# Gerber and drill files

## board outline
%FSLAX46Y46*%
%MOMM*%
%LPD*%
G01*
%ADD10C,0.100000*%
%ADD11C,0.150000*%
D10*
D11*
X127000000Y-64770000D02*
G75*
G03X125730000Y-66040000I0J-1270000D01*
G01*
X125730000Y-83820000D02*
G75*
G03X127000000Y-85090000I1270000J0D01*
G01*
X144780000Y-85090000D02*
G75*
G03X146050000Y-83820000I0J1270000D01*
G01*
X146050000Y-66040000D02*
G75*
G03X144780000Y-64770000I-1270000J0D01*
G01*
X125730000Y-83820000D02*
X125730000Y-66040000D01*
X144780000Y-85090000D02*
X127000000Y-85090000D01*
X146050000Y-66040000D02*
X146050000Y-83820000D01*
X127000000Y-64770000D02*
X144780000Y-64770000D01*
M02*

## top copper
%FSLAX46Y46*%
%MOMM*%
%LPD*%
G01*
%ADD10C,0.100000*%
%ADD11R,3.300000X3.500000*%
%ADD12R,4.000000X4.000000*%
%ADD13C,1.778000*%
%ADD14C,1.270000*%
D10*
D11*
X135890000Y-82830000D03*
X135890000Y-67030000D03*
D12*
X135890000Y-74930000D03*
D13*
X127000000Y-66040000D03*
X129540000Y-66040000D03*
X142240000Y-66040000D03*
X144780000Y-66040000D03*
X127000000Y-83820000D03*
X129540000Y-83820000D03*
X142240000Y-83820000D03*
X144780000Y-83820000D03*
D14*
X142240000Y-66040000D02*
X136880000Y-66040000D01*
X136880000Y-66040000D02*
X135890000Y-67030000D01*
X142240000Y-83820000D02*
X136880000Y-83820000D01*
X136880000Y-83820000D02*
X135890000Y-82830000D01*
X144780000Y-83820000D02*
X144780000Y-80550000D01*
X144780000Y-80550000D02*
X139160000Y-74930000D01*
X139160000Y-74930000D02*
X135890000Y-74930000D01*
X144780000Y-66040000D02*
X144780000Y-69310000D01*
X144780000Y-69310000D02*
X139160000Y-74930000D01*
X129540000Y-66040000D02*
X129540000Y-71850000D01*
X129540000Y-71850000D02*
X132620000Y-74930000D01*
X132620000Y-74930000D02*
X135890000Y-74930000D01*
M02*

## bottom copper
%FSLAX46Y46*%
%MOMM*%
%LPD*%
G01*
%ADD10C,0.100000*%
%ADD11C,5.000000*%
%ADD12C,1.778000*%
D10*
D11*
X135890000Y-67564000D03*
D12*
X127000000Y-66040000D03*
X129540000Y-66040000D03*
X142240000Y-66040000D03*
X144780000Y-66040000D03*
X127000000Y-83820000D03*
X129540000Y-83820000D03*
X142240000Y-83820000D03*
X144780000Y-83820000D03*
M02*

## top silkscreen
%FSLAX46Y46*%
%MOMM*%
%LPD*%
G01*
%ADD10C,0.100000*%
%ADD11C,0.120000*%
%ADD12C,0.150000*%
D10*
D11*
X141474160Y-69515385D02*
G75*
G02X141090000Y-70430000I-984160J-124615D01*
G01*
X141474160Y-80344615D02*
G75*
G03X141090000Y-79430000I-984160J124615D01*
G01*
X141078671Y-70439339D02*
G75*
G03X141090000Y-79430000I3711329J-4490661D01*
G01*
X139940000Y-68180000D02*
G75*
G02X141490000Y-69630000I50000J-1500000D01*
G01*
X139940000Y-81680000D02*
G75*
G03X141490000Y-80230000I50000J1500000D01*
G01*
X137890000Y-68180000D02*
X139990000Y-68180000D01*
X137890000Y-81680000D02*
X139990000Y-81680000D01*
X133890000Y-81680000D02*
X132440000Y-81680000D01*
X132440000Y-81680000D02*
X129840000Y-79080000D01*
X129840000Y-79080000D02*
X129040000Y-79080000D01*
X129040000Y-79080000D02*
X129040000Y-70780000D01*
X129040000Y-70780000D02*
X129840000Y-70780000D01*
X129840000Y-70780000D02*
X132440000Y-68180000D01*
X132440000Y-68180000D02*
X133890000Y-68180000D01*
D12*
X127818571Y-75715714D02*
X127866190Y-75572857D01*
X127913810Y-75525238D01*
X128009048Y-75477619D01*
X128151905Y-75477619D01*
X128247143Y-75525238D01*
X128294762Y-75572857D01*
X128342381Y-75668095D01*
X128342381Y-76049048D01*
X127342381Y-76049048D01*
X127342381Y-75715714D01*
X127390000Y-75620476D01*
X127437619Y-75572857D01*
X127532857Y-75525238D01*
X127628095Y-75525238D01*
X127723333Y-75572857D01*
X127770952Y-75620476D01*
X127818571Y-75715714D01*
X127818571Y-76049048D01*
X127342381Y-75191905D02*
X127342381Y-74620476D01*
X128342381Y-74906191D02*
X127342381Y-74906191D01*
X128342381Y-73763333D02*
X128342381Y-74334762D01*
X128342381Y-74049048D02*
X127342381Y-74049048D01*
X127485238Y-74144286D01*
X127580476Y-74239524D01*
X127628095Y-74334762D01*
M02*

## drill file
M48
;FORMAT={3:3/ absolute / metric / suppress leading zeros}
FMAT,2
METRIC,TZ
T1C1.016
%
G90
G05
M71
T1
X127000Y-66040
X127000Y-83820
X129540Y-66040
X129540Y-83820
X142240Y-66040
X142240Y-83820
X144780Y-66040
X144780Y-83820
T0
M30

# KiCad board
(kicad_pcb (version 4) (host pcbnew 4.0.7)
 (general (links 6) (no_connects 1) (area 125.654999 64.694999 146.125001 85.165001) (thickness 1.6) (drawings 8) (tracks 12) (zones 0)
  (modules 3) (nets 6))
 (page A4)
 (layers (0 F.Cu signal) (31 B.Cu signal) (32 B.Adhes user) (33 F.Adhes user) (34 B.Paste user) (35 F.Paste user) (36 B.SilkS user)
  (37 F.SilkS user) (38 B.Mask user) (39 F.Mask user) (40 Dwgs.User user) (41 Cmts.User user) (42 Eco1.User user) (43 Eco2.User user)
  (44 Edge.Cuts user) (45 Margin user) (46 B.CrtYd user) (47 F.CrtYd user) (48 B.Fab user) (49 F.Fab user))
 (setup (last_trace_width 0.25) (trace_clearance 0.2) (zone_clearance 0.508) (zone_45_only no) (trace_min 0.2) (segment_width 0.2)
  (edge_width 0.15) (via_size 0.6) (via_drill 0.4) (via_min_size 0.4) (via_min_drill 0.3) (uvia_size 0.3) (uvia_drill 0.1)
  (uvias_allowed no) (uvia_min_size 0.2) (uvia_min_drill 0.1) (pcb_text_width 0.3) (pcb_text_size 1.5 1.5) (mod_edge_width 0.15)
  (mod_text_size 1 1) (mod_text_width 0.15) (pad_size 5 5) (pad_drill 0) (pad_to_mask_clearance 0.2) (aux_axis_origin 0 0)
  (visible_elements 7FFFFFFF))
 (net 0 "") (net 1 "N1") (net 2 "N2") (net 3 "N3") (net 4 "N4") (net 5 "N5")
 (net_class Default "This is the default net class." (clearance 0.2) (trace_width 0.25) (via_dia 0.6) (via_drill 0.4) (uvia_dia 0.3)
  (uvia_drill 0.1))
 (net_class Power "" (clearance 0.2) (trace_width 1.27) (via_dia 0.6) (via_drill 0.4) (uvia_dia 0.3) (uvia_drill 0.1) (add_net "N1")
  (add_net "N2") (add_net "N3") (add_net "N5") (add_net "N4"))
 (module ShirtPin (layer B.Cu) (at 135.89 67.564)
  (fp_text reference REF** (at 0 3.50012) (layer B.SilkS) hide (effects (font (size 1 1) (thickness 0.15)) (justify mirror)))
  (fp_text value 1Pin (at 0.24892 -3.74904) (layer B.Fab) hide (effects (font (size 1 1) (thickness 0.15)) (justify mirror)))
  (pad 1 smd circle (at 0 0) (size 5 5) (layers B.Cu B.Mask)))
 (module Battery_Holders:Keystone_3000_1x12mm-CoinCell (layer F.Cu) (at 135.89 74.93 90)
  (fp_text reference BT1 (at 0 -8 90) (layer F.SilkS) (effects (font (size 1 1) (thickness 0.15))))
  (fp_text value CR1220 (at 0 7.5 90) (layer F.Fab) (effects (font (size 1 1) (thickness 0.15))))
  (fp_arc (start 5.29 4.6) (end 4.5 5.2) (angle -60) (layer F.SilkS) (width 0.12))
  (fp_arc (start -5.29 4.6) (end -4.5 5.2) (angle 60) (layer F.SilkS) (width 0.12))
  (fp_arc (start 0 8.9) (end -4.5 5.2) (angle 101) (layer F.SilkS) (width 0.12))
  (fp_arc (start 5.25 4.1) (end 5.3 5.6) (angle -90) (layer F.SilkS) (width 0.12))
  (fp_arc (start -5.25 4.1) (end -5.3 5.6) (angle 90) (layer F.SilkS) (width 0.12))
  (fp_line (start 6.75 2) (end 6.75 4.1) (layer F.SilkS) (width 0.12))
  (fp_line (start -6.75 2) (end -6.75 4.1) (layer F.SilkS) (width 0.12))
  (fp_line (start -6.75 -2) (end -6.75 -3.45) (layer F.SilkS) (width 0.12))
  (fp_line (start -6.75 -3.45) (end -4.15 -6.05) (layer F.SilkS) (width 0.12))
  (fp_line (start -4.15 -6.05) (end -4.15 -6.85) (layer F.SilkS) (width 0.12))
  (fp_line (start -4.15 -6.85) (end 4.15 -6.85) (layer F.SilkS) (width 0.12))
  (fp_line (start 4.15 -6.85) (end 4.15 -6.05) (layer F.SilkS) (width 0.12))
  (fp_line (start 4.15 -6.05) (end 6.75 -3.45) (layer F.SilkS) (width 0.12))
  (fp_line (start 6.75 -3.45) (end 6.75 -2) (layer F.SilkS) (width 0.12))
  (pad 1 smd rect (at -7.9 0 90) (size 3.5 3.3) (layers F.Cu F.Paste F.Mask) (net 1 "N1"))
  (pad 1 smd rect (at 7.9 0 90) (size 3.5 3.3) (layers F.Cu F.Paste F.Mask) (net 1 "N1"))
  (pad 2 smd rect (at 0 0 90) (size 4 4) (layers F.Cu F.Mask) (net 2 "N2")))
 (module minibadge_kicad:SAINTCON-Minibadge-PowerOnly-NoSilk (layer F.Cu) (at 125.73 64.77)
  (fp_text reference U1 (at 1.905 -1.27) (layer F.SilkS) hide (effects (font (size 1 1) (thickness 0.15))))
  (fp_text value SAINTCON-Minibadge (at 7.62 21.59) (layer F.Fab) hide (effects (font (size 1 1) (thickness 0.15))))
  (pad 1 thru_hole circle (at 1.27 1.27 90) (size 1.778 1.778) (drill 1.016) (layers *.Cu *.Mask) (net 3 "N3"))
  (pad 2 thru_hole circle (at 3.81 1.27 90) (size 1.778 1.778) (drill 1.016) (layers *.Cu *.Mask) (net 2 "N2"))
  (pad 7 thru_hole circle (at 16.51 1.27 90) (size 1.778 1.778) (drill 1.016) (layers *.Cu *.Mask) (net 1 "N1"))
  (pad 8 thru_hole circle (at 19.05 1.27 90) (size 1.778 1.778) (drill 1.016) (layers *.Cu *.Mask) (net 2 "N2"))
  (pad 9 thru_hole circle (at 1.27 19.05 90) (size 1.778 1.778) (drill 1.016) (layers *.Cu *.Mask) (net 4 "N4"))
  (pad 10 thru_hole circle (at 3.81 19.05 90) (size 1.778 1.778) (drill 1.016) (layers *.Cu *.Mask) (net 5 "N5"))
  (pad 15 thru_hole circle (at 16.51 19.05 90) (size 1.778 1.778) (drill 1.016) (layers *.Cu *.Mask) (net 1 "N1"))
  (pad 16 thru_hole circle (at 19.05 19.05 90) (size 1.778 1.778) (drill 1.016) (layers *.Cu *.Mask) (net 2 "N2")))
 (gr_arc (start 127 66.04) (end 125.73 66.04) (angle 90) (layer Edge.Cuts) (width 0.15))
 (gr_arc (start 127 83.82) (end 127 85.09) (angle 90) (layer Edge.Cuts) (width 0.15))
 (gr_arc (start 144.78 83.82) (end 146.05 83.82) (angle 90) (layer Edge.Cuts) (width 0.15))
 (gr_arc (start 144.78 66.04) (end 144.78 64.77) (angle 90) (layer Edge.Cuts) (width 0.15))
 (gr_line (start 125.73 83.82) (end 125.73 66.04) (layer Edge.Cuts) (width 0.15))
 (gr_line (start 144.78 85.09) (end 127 85.09) (layer Edge.Cuts) (width 0.15))
 (gr_line (start 146.05 66.04) (end 146.05 83.82) (layer Edge.Cuts) (width 0.15))
 (gr_line (start 127 64.77) (end 144.78 64.77) (layer Edge.Cuts) (width 0.15))
 (segment (start 142.24 66.04) (end 136.88 66.04) (width 1.27) (layer F.Cu) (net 1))
 (segment (start 136.88 66.04) (end 135.89 67.03) (width 1.27) (layer F.Cu) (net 1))
 (segment (start 142.24 83.82) (end 136.88 83.82) (width 1.27) (layer F.Cu) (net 1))
 (segment (start 136.88 83.82) (end 135.89 82.83) (width 1.27) (layer F.Cu) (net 1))
 (segment (start 144.78 83.82) (end 144.78 80.55) (width 1.27) (layer F.Cu) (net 2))
 (segment (start 144.78 80.55) (end 139.16 74.93) (width 1.27) (layer F.Cu) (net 2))
 (segment (start 139.16 74.93) (end 135.89 74.93) (width 1.27) (layer F.Cu) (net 2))
 (segment (start 144.78 66.04) (end 144.78 69.31) (width 1.27) (layer F.Cu) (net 2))
 (segment (start 144.78 69.31) (end 139.16 74.93) (width 1.27) (layer F.Cu) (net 2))
 (segment (start 129.54 66.04) (end 129.54 71.85) (width 1.27) (layer F.Cu) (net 2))
 (segment (start 129.54 71.85) (end 132.62 74.93) (width 1.27) (layer F.Cu) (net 2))
 (segment (start 132.62 74.93) (end 135.89 74.93) (width 1.27) (layer F.Cu) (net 2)))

